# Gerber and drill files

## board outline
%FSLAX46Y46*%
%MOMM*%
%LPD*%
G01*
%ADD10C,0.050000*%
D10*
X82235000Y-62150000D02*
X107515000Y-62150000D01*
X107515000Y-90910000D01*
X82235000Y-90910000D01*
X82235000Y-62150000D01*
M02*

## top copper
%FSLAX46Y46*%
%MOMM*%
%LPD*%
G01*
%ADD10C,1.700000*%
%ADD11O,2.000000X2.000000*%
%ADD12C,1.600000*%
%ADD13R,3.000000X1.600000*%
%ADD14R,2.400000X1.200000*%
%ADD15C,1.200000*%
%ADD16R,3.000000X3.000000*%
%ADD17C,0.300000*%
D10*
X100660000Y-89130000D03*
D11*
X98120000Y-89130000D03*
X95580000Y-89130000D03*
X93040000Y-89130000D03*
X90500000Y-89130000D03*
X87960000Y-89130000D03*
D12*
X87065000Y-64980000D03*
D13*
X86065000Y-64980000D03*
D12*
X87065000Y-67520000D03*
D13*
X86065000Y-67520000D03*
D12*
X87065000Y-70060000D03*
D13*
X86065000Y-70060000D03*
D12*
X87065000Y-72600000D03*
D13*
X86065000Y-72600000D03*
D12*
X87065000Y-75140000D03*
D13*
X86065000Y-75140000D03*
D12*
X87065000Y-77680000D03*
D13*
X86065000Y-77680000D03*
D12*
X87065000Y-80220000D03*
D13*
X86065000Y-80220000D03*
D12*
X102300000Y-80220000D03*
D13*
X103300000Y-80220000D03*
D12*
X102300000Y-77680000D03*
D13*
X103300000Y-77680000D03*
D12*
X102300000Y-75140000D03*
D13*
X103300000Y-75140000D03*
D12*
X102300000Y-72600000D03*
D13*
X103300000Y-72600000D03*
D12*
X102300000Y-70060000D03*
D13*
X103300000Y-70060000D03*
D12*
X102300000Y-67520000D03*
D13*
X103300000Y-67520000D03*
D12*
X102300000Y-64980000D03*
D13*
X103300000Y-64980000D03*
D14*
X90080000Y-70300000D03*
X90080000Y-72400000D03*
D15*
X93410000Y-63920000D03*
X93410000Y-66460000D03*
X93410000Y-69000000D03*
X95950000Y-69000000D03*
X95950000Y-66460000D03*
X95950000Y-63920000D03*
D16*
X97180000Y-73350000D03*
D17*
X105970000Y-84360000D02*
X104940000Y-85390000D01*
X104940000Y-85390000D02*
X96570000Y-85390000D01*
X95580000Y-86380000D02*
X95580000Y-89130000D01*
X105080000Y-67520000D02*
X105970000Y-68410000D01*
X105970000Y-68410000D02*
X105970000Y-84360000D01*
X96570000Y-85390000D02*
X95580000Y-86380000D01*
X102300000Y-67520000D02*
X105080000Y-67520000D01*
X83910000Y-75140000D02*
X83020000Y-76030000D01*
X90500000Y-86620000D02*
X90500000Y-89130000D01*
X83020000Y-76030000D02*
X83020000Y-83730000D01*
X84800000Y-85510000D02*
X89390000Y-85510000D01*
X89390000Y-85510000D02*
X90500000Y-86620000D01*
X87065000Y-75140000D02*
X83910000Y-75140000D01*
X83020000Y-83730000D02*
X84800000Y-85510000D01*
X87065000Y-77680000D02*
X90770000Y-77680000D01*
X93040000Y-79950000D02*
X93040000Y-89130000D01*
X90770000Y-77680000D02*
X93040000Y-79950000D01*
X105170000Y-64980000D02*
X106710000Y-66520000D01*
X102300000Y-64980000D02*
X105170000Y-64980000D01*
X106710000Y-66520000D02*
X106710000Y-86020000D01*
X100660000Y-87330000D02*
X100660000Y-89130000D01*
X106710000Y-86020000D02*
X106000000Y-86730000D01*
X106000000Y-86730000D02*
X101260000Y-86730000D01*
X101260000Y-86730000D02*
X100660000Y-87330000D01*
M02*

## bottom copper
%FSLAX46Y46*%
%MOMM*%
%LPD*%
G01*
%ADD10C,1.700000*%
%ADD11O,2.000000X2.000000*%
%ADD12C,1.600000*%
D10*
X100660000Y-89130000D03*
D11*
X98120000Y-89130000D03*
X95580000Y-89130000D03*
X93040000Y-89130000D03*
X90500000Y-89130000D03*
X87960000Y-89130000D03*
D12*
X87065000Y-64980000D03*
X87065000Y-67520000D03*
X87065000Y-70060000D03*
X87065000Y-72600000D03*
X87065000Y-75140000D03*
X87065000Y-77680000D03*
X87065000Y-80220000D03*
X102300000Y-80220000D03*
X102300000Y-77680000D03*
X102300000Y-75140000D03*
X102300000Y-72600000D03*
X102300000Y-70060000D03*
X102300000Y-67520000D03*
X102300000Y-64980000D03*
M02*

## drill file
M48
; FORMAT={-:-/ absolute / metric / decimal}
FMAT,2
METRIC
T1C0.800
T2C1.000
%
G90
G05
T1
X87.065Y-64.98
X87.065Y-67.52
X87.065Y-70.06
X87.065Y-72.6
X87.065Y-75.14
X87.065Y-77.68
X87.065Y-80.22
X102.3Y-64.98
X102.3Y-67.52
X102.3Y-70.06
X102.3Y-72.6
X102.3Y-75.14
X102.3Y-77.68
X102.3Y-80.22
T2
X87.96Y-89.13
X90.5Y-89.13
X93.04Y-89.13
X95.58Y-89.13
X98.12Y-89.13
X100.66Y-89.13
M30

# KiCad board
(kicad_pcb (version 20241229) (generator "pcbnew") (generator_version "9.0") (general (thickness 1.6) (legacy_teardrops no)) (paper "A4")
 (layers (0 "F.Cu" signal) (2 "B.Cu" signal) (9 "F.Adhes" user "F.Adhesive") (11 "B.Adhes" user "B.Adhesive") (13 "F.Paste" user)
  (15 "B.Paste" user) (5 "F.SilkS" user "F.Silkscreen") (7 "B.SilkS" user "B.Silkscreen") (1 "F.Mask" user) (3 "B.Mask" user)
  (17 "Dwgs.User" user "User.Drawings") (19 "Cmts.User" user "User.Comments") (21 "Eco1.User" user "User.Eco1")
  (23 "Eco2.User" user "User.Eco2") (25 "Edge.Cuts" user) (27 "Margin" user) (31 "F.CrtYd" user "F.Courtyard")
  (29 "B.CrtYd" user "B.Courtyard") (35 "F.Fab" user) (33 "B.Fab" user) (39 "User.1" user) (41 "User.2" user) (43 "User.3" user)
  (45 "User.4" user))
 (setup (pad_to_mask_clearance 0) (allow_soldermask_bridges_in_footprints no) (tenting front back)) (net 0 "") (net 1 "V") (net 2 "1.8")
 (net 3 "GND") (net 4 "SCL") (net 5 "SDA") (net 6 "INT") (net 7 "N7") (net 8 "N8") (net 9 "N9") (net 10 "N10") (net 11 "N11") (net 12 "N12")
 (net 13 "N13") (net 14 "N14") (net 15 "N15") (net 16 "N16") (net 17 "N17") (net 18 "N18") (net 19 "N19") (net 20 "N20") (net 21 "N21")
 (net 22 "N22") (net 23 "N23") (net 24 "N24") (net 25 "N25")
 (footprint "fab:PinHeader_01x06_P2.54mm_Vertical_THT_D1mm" (layer "F.Cu") (at 100.66 89.13 -90)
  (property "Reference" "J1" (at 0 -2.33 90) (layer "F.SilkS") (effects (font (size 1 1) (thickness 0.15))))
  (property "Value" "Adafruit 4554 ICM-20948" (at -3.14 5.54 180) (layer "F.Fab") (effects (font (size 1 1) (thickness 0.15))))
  (pad "1" thru_hole circle (at 0 0 270) (size 1.7 1.7) (drill 1) (layers "*.Cu" "*.Mask") (remove_unused_layers no) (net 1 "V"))
  (pad "2" thru_hole oval (at 0 2.54 270) (size 2 2) (drill 1) (layers "*.Cu" "*.Mask") (remove_unused_layers no) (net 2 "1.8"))
  (pad "3" thru_hole oval (at 0 5.08 270) (size 2 2) (drill 1) (layers "*.Cu" "*.Mask") (remove_unused_layers no) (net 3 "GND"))
  (pad "4" thru_hole oval (at 0 7.62 270) (size 2 2) (drill 1) (layers "*.Cu" "*.Mask") (remove_unused_layers no) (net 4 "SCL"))
  (pad "5" thru_hole oval (at 0 10.16 270) (size 2 2) (drill 1) (layers "*.Cu" "*.Mask") (remove_unused_layers no) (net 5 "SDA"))
  (pad "6" thru_hole oval (at 0 12.7 270) (size 2 2) (drill 1) (layers "*.Cu" "*.Mask") (remove_unused_layers no) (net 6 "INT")))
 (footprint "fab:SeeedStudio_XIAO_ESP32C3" (layer "F.Cu") (at 94.68 72.6)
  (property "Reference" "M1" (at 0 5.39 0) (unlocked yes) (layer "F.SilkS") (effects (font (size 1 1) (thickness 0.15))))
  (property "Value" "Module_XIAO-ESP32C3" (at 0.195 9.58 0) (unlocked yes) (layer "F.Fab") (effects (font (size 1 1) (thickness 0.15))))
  (pad "1" thru_hole circle (at -7.615 -7.62) (size 1.6 1.6) (drill 0.8) (layers "*.Cu" "*.Mask") (remove_unused_layers no) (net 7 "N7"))
  (pad "1" smd rect (at -7.615 -7.62) (size 3 1.6) (drill (offset -1 0)) (layers "F.Cu" "F.Mask" "F.Paste") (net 7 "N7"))
  (pad "2" thru_hole circle (at -7.615 -5.08) (size 1.6 1.6) (drill 0.8) (layers "*.Cu" "*.Mask") (remove_unused_layers no) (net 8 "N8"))
  (pad "2" smd rect (at -7.615 -5.08) (size 3 1.6) (drill (offset -1 0)) (layers "F.Cu" "F.Mask" "F.Paste") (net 8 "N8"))
  (pad "3" thru_hole circle (at -7.615 -2.54) (size 1.6 1.6) (drill 0.8) (layers "*.Cu" "*.Mask") (remove_unused_layers no) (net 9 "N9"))
  (pad "3" smd rect (at -7.615 -2.54) (size 3 1.6) (drill (offset -1 0)) (layers "F.Cu" "F.Mask" "F.Paste") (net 9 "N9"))
  (pad "4" thru_hole circle (at -7.615 0) (size 1.6 1.6) (drill 0.8) (layers "*.Cu" "*.Mask") (remove_unused_layers no) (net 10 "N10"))
  (pad "4" smd rect (at -7.615 0) (size 3 1.6) (drill (offset -1 0)) (layers "F.Cu" "F.Mask" "F.Paste") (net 10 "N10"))
  (pad "5" thru_hole circle (at -7.615 2.54) (size 1.6 1.6) (drill 0.8) (layers "*.Cu" "*.Mask") (remove_unused_layers no) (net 5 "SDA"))
  (pad "5" smd rect (at -7.615 2.54) (size 3 1.6) (drill (offset -1 0)) (layers "F.Cu" "F.Mask" "F.Paste") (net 5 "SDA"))
  (pad "6" thru_hole circle (at -7.615 5.08) (size 1.6 1.6) (drill 0.8) (layers "*.Cu" "*.Mask") (remove_unused_layers no) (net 4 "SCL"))
  (pad "6" smd rect (at -7.615 5.08) (size 3 1.6) (drill (offset -1 0)) (layers "F.Cu" "F.Mask" "F.Paste") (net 4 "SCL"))
  (pad "7" thru_hole circle (at -7.615 7.62) (size 1.6 1.6) (drill 0.8) (layers "*.Cu" "*.Mask") (remove_unused_layers no) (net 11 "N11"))
  (pad "7" smd rect (at -7.615 7.62) (size 3 1.6) (drill (offset -1 0)) (layers "F.Cu" "F.Mask" "F.Paste") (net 11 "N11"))
  (pad "8" thru_hole circle (at 7.62 7.62) (size 1.6 1.6) (drill 0.8) (layers "*.Cu" "*.Mask") (remove_unused_layers no) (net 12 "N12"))
  (pad "8" smd rect (at 7.62 7.62) (size 3 1.6) (drill (offset 1 0)) (layers "F.Cu" "F.Mask" "F.Paste") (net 12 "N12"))
  (pad "9" thru_hole circle (at 7.62 5.08) (size 1.6 1.6) (drill 0.8) (layers "*.Cu" "*.Mask") (remove_unused_layers no) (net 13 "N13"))
  (pad "9" smd rect (at 7.62 5.08) (size 3 1.6) (drill (offset 1 0)) (layers "F.Cu" "F.Mask" "F.Paste") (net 13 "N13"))
  (pad "10" thru_hole circle (at 7.62 2.54) (size 1.6 1.6) (drill 0.8) (layers "*.Cu" "*.Mask") (remove_unused_layers no) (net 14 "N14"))
  (pad "10" smd rect (at 7.62 2.54) (size 3 1.6) (drill (offset 1 0)) (layers "F.Cu" "F.Mask" "F.Paste") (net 14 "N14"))
  (pad "11" thru_hole circle (at 7.62 0) (size 1.6 1.6) (drill 0.8) (layers "*.Cu" "*.Mask") (remove_unused_layers no) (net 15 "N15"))
  (pad "11" smd rect (at 7.62 0) (size 3 1.6) (drill (offset 1 0)) (layers "F.Cu" "F.Mask" "F.Paste") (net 15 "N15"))
  (pad "12" thru_hole circle (at 7.62 -2.54) (size 1.6 1.6) (drill 0.8) (layers "*.Cu" "*.Mask") (remove_unused_layers no) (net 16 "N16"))
  (pad "12" smd rect (at 7.62 -2.54) (size 3 1.6) (drill (offset 1 0)) (layers "F.Cu" "F.Mask" "F.Paste") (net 16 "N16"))
  (pad "13" thru_hole circle (at 7.62 -5.08) (size 1.6 1.6) (drill 0.8) (layers "*.Cu" "*.Mask") (remove_unused_layers no) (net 3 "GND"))
  (pad "13" smd rect (at 7.62 -5.08) (size 3 1.6) (drill (offset 1 0)) (layers "F.Cu" "F.Mask" "F.Paste") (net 3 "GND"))
  (pad "14" thru_hole circle (at 7.62 -7.62) (size 1.6 1.6) (drill 0.8) (layers "*.Cu" "*.Mask") (remove_unused_layers no) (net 1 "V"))
  (pad "14" smd rect (at 7.62 -7.62) (size 3 1.6) (drill (offset 1 0)) (layers "F.Cu" "F.Mask" "F.Paste") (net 1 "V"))
  (pad "15" smd rect (at -4.6 -2.3) (size 2.4 1.2) (layers "F.Cu" "F.Mask" "F.Paste") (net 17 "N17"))
  (pad "16" smd rect (at -4.6 -0.2) (size 2.4 1.2) (layers "F.Cu" "F.Mask" "F.Paste") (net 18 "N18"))
  (pad "17" smd circle (at -1.27 -8.68) (size 1.2 1.2) (layers "F.Cu" "F.Mask" "F.Paste") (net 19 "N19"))
  (pad "18" smd circle (at -1.27 -6.14) (size 1.2 1.2) (layers "F.Cu" "F.Mask" "F.Paste") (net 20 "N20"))
  (pad "19" smd circle (at -1.27 -3.6) (size 1.2 1.2) (layers "F.Cu" "F.Mask" "F.Paste") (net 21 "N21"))
  (pad "20" smd circle (at 1.27 -3.6) (size 1.2 1.2) (layers "F.Cu" "F.Mask" "F.Paste") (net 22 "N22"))
  (pad "21" smd circle (at 1.27 -6.14) (size 1.2 1.2) (layers "F.Cu" "F.Mask" "F.Paste") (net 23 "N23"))
  (pad "22" smd circle (at 1.27 -8.68) (size 1.2 1.2) (layers "F.Cu" "F.Mask" "F.Paste") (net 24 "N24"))
  (pad "23" smd rect (at 2.5 0.75) (size 3 3) (layers "F.Cu" "F.Mask" "F.Paste") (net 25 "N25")))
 (gr_rect (start 82.235 62.15) (end 107.515 90.91) (stroke (width 0.05) (type default)) (fill no) (layer "Edge.Cuts"))
 (segment (start 105.97 84.36) (end 104.94 85.39) (width 0.3) (layer "F.Cu") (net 3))
 (segment (start 104.94 85.39) (end 96.57 85.39) (width 0.3) (layer "F.Cu") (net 3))
 (segment (start 95.58 86.38) (end 95.58 89.13) (width 0.3) (layer "F.Cu") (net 3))
 (segment (start 105.08 67.52) (end 105.97 68.41) (width 0.3) (layer "F.Cu") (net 3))
 (segment (start 105.97 68.41) (end 105.97 84.36) (width 0.3) (layer "F.Cu") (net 3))
 (segment (start 96.57 85.39) (end 95.58 86.38) (width 0.3) (layer "F.Cu") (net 3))
 (segment (start 102.3 67.52) (end 105.08 67.52) (width 0.3) (layer "F.Cu") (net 3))
 (segment (start 83.91 75.14) (end 83.02 76.03) (width 0.3) (layer "F.Cu") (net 5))
 (segment (start 90.5 86.62) (end 90.5 89.13) (width 0.3) (layer "F.Cu") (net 5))
 (segment (start 83.02 76.03) (end 83.02 83.73) (width 0.3) (layer "F.Cu") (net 5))
 (segment (start 84.8 85.51) (end 89.39 85.51) (width 0.3) (layer "F.Cu") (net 5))
 (segment (start 89.39 85.51) (end 90.5 86.62) (width 0.3) (layer "F.Cu") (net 5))
 (segment (start 87.065 75.14) (end 83.91 75.14) (width 0.3) (layer "F.Cu") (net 5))
 (segment (start 83.02 83.73) (end 84.8 85.51) (width 0.3) (layer "F.Cu") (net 5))
 (segment (start 87.065 77.68) (end 90.77 77.68) (width 0.3) (layer "F.Cu") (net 4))
 (segment (start 93.04 79.95) (end 93.04 89.13) (width 0.3) (layer "F.Cu") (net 4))
 (segment (start 90.77 77.68) (end 93.04 79.95) (width 0.3) (layer "F.Cu") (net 4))
 (segment (start 105.17 64.98) (end 106.71 66.52) (width 0.3) (layer "F.Cu") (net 1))
 (segment (start 102.3 64.98) (end 105.17 64.98) (width 0.3) (layer "F.Cu") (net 1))
 (segment (start 106.71 66.52) (end 106.71 86.02) (width 0.3) (layer "F.Cu") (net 1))
 (segment (start 100.66 87.33) (end 100.66 89.13) (width 0.3) (layer "F.Cu") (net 1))
 (segment (start 106.71 86.02) (end 106 86.73) (width 0.3) (layer "F.Cu") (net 1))
 (segment (start 106 86.73) (end 101.26 86.73) (width 0.3) (layer "F.Cu") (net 1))
 (segment (start 101.26 86.73) (end 100.66 87.33) (width 0.3) (layer "F.Cu") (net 1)))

